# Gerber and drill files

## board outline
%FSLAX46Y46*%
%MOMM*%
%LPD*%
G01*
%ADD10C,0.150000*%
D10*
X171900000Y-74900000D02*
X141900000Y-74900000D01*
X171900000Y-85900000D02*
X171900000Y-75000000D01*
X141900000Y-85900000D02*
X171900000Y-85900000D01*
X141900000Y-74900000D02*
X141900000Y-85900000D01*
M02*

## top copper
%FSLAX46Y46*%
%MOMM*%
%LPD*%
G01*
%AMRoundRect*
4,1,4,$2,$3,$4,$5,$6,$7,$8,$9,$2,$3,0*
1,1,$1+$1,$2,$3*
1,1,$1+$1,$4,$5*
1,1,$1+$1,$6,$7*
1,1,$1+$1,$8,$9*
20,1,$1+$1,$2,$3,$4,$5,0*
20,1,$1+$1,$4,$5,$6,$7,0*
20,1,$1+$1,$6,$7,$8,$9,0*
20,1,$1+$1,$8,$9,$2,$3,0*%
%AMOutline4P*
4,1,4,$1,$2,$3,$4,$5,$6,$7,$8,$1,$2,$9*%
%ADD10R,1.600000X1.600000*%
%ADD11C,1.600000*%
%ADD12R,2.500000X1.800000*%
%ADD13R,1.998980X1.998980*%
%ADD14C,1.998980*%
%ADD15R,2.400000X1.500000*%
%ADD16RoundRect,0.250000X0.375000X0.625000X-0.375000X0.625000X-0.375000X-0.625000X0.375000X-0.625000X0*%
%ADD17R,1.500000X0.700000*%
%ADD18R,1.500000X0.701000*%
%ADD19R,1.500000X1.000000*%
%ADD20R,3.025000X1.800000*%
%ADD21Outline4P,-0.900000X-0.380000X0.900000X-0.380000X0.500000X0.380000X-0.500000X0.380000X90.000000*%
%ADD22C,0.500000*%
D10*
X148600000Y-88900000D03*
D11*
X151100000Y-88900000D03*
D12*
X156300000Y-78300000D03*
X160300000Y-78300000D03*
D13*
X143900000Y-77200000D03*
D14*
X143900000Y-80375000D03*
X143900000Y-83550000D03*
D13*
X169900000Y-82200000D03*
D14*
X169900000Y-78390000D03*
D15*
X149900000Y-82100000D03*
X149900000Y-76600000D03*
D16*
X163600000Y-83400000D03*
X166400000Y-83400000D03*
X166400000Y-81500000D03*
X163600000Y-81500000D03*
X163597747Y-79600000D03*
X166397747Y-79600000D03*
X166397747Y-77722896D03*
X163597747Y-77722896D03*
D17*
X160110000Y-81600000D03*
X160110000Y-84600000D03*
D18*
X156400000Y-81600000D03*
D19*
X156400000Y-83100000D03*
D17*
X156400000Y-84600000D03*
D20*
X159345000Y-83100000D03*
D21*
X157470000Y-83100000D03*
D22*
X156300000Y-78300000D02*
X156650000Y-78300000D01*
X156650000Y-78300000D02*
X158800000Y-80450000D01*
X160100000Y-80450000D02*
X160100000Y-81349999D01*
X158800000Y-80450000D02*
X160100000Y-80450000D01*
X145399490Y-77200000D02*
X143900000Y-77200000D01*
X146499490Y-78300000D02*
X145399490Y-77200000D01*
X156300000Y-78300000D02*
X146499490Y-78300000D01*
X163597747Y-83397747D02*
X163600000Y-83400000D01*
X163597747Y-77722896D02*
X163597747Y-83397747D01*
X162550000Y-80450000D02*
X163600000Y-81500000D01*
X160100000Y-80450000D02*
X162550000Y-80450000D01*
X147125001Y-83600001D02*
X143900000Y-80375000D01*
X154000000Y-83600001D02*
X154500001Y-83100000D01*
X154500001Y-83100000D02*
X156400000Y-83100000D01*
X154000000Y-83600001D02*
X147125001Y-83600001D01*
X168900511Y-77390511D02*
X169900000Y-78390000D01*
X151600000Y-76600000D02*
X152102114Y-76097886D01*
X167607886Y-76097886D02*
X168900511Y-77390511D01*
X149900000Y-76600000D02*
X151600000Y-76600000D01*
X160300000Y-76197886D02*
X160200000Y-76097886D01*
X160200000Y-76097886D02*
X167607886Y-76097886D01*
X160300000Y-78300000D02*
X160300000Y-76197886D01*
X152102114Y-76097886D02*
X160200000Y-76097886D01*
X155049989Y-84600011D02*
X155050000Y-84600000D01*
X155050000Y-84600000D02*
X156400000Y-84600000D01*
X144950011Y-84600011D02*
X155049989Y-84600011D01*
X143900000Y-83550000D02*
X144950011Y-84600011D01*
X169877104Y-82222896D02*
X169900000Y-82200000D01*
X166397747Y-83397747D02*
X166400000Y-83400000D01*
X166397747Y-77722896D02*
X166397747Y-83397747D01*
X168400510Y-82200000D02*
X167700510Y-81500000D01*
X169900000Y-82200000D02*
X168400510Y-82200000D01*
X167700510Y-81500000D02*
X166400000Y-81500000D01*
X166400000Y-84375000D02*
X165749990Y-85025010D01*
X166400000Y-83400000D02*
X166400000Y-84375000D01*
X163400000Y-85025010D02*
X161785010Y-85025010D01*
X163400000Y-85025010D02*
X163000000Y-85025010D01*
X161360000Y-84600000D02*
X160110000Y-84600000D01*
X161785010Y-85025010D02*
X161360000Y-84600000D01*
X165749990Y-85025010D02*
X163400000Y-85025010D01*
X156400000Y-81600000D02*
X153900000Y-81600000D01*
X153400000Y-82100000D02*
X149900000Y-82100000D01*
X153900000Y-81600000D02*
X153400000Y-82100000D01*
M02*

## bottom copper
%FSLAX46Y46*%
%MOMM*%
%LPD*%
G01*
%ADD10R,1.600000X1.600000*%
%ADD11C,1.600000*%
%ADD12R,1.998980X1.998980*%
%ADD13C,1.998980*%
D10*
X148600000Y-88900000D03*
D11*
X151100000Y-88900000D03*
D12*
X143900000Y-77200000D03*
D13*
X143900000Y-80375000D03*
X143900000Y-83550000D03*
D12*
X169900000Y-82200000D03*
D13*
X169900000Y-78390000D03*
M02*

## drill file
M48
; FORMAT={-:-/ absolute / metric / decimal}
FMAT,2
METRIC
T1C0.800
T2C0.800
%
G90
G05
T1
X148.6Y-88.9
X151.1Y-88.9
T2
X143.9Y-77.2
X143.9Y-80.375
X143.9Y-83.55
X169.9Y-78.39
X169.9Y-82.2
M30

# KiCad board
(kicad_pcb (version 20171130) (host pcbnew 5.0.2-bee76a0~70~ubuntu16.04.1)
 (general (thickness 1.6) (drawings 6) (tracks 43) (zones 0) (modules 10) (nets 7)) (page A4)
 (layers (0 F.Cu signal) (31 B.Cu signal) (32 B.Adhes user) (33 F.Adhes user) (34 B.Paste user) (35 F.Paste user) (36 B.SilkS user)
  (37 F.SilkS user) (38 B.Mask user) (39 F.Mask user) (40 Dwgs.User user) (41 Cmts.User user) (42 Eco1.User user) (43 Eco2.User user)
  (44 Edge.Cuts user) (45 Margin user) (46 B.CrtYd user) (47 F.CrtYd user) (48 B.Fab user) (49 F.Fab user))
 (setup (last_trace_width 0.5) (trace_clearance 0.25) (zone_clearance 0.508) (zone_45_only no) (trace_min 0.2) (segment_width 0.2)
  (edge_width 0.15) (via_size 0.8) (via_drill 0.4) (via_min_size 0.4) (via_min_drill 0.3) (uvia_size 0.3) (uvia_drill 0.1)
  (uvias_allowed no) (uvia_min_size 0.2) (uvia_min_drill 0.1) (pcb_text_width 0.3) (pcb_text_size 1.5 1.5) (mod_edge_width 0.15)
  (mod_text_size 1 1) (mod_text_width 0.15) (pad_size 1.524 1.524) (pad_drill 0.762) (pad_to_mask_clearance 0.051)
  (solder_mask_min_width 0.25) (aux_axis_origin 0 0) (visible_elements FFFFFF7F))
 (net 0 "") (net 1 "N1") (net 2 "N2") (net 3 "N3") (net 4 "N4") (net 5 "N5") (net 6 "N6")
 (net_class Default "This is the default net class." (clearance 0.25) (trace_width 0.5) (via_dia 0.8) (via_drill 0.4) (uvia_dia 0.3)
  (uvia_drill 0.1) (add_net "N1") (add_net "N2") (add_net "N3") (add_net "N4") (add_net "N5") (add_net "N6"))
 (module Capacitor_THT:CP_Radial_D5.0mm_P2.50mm (layer F.Cu) (at 148.6 88.9)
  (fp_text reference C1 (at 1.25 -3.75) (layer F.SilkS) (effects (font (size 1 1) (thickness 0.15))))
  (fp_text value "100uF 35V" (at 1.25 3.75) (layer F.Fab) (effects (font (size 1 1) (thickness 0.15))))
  (pad 1 thru_hole rect (at 0 0) (size 1.6 1.6) (drill 0.8) (layers *.Cu *.Mask) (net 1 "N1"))
  (pad 2 thru_hole circle (at 2.5 0) (size 1.6 1.6) (drill 0.8) (layers *.Cu *.Mask) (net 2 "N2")))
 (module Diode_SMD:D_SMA (layer F.Cu) (at 158.3 78.3)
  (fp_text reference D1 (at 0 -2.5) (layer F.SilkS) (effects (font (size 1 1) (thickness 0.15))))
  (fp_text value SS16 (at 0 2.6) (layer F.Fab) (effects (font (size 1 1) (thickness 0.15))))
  (pad 1 smd rect (at -2 0) (size 2.5 1.8) (layers F.Cu F.Paste F.Mask) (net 1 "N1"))
  (pad 2 smd rect (at 2 0) (size 2.5 1.8) (layers F.Cu F.Paste F.Mask) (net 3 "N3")))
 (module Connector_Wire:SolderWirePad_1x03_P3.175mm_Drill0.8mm (layer F.Cu) (at 143.9 77.2 270)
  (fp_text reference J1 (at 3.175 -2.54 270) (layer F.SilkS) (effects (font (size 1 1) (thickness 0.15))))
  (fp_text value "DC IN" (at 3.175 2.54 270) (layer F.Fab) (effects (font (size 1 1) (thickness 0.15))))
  (pad 1 thru_hole rect (at 0 0 270) (size 1.99898 1.99898) (drill 0.8001) (layers *.Cu *.Mask) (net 1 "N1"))
  (pad 2 thru_hole circle (at 3.175 0 270) (size 1.99898 1.99898) (drill 0.8001) (layers *.Cu *.Mask) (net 2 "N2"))
  (pad 3 thru_hole circle (at 6.35 0 270) (size 1.99898 1.99898) (drill 0.8001) (layers *.Cu *.Mask) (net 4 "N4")))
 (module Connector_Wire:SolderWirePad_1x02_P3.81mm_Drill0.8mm (layer F.Cu) (at 169.9 82.2 90)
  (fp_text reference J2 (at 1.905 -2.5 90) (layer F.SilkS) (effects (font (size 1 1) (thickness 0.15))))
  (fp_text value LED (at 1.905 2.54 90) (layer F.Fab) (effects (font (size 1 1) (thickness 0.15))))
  (pad 1 thru_hole rect (at 0 0 90) (size 1.99898 1.99898) (drill 0.8001) (layers *.Cu *.Mask) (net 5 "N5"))
  (pad 2 thru_hole circle (at 3.81 0 90) (size 1.99898 1.99898) (drill 0.8001) (layers *.Cu *.Mask) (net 3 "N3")))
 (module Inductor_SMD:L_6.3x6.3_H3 (layer F.Cu) (at 149.9 79.35 90)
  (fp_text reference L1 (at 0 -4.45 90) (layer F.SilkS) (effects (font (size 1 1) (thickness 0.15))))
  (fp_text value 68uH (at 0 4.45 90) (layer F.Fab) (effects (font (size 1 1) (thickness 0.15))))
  (pad 1 smd rect (at -2.75 0 90) (size 1.5 2.4) (layers F.Cu F.Paste F.Mask) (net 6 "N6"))
  (pad 2 smd rect (at 2.75 0 90) (size 1.5 2.4) (layers F.Cu F.Paste F.Mask) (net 3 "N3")))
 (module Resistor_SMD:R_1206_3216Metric (layer F.Cu) (at 165 83.4 180)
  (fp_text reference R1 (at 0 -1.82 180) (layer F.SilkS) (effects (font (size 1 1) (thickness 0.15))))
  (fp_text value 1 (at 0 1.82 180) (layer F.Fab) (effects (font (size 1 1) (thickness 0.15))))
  (pad 2 smd roundrect (at 1.4 0 180) (size 1.25 1.75) (layers F.Cu F.Paste F.Mask) (roundrect_rratio 0.2) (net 1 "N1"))
  (pad 1 smd roundrect (at -1.4 0 180) (size 1.25 1.75) (layers F.Cu F.Paste F.Mask) (roundrect_rratio 0.2) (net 5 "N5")))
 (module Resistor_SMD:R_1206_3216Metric (layer F.Cu) (at 165 81.5 180)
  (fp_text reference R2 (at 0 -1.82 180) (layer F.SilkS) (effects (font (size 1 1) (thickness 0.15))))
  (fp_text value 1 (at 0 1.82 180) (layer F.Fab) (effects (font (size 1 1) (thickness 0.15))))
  (pad 1 smd roundrect (at -1.4 0 180) (size 1.25 1.75) (layers F.Cu F.Paste F.Mask) (roundrect_rratio 0.2) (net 5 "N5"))
  (pad 2 smd roundrect (at 1.4 0 180) (size 1.25 1.75) (layers F.Cu F.Paste F.Mask) (roundrect_rratio 0.2) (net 1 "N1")))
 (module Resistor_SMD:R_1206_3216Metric (layer F.Cu) (at 164.997747 79.6 180)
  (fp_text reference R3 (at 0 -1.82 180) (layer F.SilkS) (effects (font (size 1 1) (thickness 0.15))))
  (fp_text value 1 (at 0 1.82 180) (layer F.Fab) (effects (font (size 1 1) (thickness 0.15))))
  (pad 2 smd roundrect (at 1.4 0 180) (size 1.25 1.75) (layers F.Cu F.Paste F.Mask) (roundrect_rratio 0.2) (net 1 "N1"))
  (pad 1 smd roundrect (at -1.4 0 180) (size 1.25 1.75) (layers F.Cu F.Paste F.Mask) (roundrect_rratio 0.2) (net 5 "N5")))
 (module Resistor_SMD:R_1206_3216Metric (layer F.Cu) (at 164.997747 77.722896 180)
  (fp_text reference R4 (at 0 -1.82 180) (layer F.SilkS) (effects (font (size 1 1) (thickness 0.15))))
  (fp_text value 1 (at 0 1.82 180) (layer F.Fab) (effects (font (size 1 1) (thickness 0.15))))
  (pad 1 smd roundrect (at -1.4 0 180) (size 1.25 1.75) (layers F.Cu F.Paste F.Mask) (roundrect_rratio 0.2) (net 5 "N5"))
  (pad 2 smd roundrect (at 1.4 0 180) (size 1.25 1.75) (layers F.Cu F.Paste F.Mask) (roundrect_rratio 0.2) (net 1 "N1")))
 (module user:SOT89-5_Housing (layer F.Cu) (at 158.25 83.1 270)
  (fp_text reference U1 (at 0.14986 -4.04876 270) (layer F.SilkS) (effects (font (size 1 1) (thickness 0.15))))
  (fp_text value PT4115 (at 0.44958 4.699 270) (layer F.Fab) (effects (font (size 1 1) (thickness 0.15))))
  (pad 5 smd rect (at -1.5 -1.86 270) (size 0.7 1.5) (layers F.Cu F.Paste F.Mask) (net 1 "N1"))
  (pad 4 smd rect (at 1.5 -1.86 270) (size 0.7 1.5) (layers F.Cu F.Paste F.Mask) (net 5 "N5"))
  (pad 1 smd rect (at -1.5 1.85 270) (size 0.701 1.5) (layers F.Cu F.Paste F.Mask) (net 6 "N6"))
  (pad 2 smd rect (at 0 1.85 270) (size 1 1.5) (layers F.Cu F.Paste F.Mask) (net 2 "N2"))
  (pad 3 smd rect (at 1.5 1.85 270) (size 0.7 1.5) (layers F.Cu F.Paste F.Mask) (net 4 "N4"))
  (pad 2 smd rect (at 0 -1.095 270) (size 1.8 3.025) (layers F.Cu F.Paste F.Mask) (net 2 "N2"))
  (pad 2 smd trapezoid (at 0 0.78 90) (size 1.4 0.76) (rect_delta 0 0.4) (layers F.Cu F.Paste F.Mask) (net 2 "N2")))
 (gr_line (start 171.9 74.9) (end 141.9 74.9) (layer Edge.Cuts) (width 0.15))
 (gr_line (start 171.9 85.9) (end 171.9 75) (layer Edge.Cuts) (width 0.15))
 (gr_line (start 141.9 85.9) (end 171.9 85.9) (layer Edge.Cuts) (width 0.15))
 (gr_line (start 141.9 74.9) (end 141.9 85.9) (layer Edge.Cuts) (width 0.15))
 (segment (start 156.3 78.3) (end 156.65 78.3) (width 0.5) (layer F.Cu) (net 1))
 (segment (start 156.65 78.3) (end 158.8 80.45) (width 0.5) (layer F.Cu) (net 1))
 (segment (start 160.1 80.45) (end 160.1 81.349999) (width 0.5) (layer F.Cu) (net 1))
 (segment (start 158.8 80.45) (end 160.1 80.45) (width 0.5) (layer F.Cu) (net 1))
 (segment (start 145.39949 77.2) (end 143.9 77.2) (width 0.5) (layer F.Cu) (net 1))
 (segment (start 146.49949 78.3) (end 145.39949 77.2) (width 0.5) (layer F.Cu) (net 1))
 (segment (start 156.3 78.3) (end 146.49949 78.3) (width 0.5) (layer F.Cu) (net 1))
 (segment (start 163.597747 83.397747) (end 163.6 83.4) (width 0.5) (layer F.Cu) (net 1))
 (segment (start 163.597747 77.722896) (end 163.597747 83.397747) (width 0.5) (layer F.Cu) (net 1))
 (segment (start 162.55 80.45) (end 163.6 81.5) (width 0.5) (layer F.Cu) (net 1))
 (segment (start 160.1 80.45) (end 162.55 80.45) (width 0.5) (layer F.Cu) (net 1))
 (segment (start 147.125001 83.600001) (end 143.9 80.375) (width 0.5) (layer F.Cu) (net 2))
 (segment (start 154 83.600001) (end 154.500001 83.1) (width 0.5) (layer F.Cu) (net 2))
 (segment (start 154.500001 83.1) (end 156.4 83.1) (width 0.5) (layer F.Cu) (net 2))
 (segment (start 154 83.600001) (end 147.125001 83.600001) (width 0.5) (layer F.Cu) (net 2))
 (segment (start 168.900511 77.390511) (end 169.9 78.39) (width 0.5) (layer F.Cu) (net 3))
 (segment (start 151.6 76.6) (end 152.102114 76.097886) (width 0.5) (layer F.Cu) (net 3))
 (segment (start 167.607886 76.097886) (end 168.900511 77.390511) (width 0.5) (layer F.Cu) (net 3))
 (segment (start 149.9 76.6) (end 151.6 76.6) (width 0.5) (layer F.Cu) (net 3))
 (segment (start 160.3 76.197886) (end 160.2 76.097886) (width 0.5) (layer F.Cu) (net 3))
 (segment (start 160.2 76.097886) (end 167.607886 76.097886) (width 0.5) (layer F.Cu) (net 3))
 (segment (start 160.3 78.3) (end 160.3 76.197886) (width 0.5) (layer F.Cu) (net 3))
 (segment (start 152.102114 76.097886) (end 160.2 76.097886) (width 0.5) (layer F.Cu) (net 3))
 (segment (start 155.049989 84.600011) (end 155.05 84.6) (width 0.5) (layer F.Cu) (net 4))
 (segment (start 155.05 84.6) (end 156.4 84.6) (width 0.5) (layer F.Cu) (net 4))
 (segment (start 144.950011 84.600011) (end 155.049989 84.600011) (width 0.5) (layer F.Cu) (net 4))
 (segment (start 143.9 83.55) (end 144.950011 84.600011) (width 0.5) (layer F.Cu) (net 4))
 (segment (start 169.877104 82.222896) (end 169.9 82.2) (width 0.5) (layer F.Cu) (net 5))
 (segment (start 166.397747 83.397747) (end 166.4 83.4) (width 0.5) (layer F.Cu) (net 5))
 (segment (start 166.397747 77.722896) (end 166.397747 83.397747) (width 0.5) (layer F.Cu) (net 5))
 (segment (start 168.40051 82.2) (end 167.70051 81.5) (width 0.5) (layer F.Cu) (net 5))
 (segment (start 169.9 82.2) (end 168.40051 82.2) (width 0.5) (layer F.Cu) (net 5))
 (segment (start 167.70051 81.5) (end 166.4 81.5) (width 0.5) (layer F.Cu) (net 5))
 (segment (start 166.4 84.375) (end 165.74999 85.02501) (width 0.5) (layer F.Cu) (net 5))
 (segment (start 166.4 83.4) (end 166.4 84.375) (width 0.5) (layer F.Cu) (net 5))
 (segment (start 163.4 85.02501) (end 161.78501 85.02501) (width 0.5) (layer F.Cu) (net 5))
 (segment (start 163.4 85.02501) (end 163 85.02501) (width 0.5) (layer F.Cu) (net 5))
 (segment (start 161.36 84.6) (end 160.11 84.6) (width 0.5) (layer F.Cu) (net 5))
 (segment (start 161.78501 85.02501) (end 161.36 84.6) (width 0.5) (layer F.Cu) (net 5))
 (segment (start 165.74999 85.02501) (end 163.4 85.02501) (width 0.5) (layer F.Cu) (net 5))
 (segment (start 156.4 81.6) (end 153.9 81.6) (width 0.5) (layer F.Cu) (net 6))
 (segment (start 153.4 82.1) (end 149.9 82.1) (width 0.5) (layer F.Cu) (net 6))
 (segment (start 153.9 81.6) (end 153.4 82.1) (width 0.5) (layer F.Cu) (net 6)))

